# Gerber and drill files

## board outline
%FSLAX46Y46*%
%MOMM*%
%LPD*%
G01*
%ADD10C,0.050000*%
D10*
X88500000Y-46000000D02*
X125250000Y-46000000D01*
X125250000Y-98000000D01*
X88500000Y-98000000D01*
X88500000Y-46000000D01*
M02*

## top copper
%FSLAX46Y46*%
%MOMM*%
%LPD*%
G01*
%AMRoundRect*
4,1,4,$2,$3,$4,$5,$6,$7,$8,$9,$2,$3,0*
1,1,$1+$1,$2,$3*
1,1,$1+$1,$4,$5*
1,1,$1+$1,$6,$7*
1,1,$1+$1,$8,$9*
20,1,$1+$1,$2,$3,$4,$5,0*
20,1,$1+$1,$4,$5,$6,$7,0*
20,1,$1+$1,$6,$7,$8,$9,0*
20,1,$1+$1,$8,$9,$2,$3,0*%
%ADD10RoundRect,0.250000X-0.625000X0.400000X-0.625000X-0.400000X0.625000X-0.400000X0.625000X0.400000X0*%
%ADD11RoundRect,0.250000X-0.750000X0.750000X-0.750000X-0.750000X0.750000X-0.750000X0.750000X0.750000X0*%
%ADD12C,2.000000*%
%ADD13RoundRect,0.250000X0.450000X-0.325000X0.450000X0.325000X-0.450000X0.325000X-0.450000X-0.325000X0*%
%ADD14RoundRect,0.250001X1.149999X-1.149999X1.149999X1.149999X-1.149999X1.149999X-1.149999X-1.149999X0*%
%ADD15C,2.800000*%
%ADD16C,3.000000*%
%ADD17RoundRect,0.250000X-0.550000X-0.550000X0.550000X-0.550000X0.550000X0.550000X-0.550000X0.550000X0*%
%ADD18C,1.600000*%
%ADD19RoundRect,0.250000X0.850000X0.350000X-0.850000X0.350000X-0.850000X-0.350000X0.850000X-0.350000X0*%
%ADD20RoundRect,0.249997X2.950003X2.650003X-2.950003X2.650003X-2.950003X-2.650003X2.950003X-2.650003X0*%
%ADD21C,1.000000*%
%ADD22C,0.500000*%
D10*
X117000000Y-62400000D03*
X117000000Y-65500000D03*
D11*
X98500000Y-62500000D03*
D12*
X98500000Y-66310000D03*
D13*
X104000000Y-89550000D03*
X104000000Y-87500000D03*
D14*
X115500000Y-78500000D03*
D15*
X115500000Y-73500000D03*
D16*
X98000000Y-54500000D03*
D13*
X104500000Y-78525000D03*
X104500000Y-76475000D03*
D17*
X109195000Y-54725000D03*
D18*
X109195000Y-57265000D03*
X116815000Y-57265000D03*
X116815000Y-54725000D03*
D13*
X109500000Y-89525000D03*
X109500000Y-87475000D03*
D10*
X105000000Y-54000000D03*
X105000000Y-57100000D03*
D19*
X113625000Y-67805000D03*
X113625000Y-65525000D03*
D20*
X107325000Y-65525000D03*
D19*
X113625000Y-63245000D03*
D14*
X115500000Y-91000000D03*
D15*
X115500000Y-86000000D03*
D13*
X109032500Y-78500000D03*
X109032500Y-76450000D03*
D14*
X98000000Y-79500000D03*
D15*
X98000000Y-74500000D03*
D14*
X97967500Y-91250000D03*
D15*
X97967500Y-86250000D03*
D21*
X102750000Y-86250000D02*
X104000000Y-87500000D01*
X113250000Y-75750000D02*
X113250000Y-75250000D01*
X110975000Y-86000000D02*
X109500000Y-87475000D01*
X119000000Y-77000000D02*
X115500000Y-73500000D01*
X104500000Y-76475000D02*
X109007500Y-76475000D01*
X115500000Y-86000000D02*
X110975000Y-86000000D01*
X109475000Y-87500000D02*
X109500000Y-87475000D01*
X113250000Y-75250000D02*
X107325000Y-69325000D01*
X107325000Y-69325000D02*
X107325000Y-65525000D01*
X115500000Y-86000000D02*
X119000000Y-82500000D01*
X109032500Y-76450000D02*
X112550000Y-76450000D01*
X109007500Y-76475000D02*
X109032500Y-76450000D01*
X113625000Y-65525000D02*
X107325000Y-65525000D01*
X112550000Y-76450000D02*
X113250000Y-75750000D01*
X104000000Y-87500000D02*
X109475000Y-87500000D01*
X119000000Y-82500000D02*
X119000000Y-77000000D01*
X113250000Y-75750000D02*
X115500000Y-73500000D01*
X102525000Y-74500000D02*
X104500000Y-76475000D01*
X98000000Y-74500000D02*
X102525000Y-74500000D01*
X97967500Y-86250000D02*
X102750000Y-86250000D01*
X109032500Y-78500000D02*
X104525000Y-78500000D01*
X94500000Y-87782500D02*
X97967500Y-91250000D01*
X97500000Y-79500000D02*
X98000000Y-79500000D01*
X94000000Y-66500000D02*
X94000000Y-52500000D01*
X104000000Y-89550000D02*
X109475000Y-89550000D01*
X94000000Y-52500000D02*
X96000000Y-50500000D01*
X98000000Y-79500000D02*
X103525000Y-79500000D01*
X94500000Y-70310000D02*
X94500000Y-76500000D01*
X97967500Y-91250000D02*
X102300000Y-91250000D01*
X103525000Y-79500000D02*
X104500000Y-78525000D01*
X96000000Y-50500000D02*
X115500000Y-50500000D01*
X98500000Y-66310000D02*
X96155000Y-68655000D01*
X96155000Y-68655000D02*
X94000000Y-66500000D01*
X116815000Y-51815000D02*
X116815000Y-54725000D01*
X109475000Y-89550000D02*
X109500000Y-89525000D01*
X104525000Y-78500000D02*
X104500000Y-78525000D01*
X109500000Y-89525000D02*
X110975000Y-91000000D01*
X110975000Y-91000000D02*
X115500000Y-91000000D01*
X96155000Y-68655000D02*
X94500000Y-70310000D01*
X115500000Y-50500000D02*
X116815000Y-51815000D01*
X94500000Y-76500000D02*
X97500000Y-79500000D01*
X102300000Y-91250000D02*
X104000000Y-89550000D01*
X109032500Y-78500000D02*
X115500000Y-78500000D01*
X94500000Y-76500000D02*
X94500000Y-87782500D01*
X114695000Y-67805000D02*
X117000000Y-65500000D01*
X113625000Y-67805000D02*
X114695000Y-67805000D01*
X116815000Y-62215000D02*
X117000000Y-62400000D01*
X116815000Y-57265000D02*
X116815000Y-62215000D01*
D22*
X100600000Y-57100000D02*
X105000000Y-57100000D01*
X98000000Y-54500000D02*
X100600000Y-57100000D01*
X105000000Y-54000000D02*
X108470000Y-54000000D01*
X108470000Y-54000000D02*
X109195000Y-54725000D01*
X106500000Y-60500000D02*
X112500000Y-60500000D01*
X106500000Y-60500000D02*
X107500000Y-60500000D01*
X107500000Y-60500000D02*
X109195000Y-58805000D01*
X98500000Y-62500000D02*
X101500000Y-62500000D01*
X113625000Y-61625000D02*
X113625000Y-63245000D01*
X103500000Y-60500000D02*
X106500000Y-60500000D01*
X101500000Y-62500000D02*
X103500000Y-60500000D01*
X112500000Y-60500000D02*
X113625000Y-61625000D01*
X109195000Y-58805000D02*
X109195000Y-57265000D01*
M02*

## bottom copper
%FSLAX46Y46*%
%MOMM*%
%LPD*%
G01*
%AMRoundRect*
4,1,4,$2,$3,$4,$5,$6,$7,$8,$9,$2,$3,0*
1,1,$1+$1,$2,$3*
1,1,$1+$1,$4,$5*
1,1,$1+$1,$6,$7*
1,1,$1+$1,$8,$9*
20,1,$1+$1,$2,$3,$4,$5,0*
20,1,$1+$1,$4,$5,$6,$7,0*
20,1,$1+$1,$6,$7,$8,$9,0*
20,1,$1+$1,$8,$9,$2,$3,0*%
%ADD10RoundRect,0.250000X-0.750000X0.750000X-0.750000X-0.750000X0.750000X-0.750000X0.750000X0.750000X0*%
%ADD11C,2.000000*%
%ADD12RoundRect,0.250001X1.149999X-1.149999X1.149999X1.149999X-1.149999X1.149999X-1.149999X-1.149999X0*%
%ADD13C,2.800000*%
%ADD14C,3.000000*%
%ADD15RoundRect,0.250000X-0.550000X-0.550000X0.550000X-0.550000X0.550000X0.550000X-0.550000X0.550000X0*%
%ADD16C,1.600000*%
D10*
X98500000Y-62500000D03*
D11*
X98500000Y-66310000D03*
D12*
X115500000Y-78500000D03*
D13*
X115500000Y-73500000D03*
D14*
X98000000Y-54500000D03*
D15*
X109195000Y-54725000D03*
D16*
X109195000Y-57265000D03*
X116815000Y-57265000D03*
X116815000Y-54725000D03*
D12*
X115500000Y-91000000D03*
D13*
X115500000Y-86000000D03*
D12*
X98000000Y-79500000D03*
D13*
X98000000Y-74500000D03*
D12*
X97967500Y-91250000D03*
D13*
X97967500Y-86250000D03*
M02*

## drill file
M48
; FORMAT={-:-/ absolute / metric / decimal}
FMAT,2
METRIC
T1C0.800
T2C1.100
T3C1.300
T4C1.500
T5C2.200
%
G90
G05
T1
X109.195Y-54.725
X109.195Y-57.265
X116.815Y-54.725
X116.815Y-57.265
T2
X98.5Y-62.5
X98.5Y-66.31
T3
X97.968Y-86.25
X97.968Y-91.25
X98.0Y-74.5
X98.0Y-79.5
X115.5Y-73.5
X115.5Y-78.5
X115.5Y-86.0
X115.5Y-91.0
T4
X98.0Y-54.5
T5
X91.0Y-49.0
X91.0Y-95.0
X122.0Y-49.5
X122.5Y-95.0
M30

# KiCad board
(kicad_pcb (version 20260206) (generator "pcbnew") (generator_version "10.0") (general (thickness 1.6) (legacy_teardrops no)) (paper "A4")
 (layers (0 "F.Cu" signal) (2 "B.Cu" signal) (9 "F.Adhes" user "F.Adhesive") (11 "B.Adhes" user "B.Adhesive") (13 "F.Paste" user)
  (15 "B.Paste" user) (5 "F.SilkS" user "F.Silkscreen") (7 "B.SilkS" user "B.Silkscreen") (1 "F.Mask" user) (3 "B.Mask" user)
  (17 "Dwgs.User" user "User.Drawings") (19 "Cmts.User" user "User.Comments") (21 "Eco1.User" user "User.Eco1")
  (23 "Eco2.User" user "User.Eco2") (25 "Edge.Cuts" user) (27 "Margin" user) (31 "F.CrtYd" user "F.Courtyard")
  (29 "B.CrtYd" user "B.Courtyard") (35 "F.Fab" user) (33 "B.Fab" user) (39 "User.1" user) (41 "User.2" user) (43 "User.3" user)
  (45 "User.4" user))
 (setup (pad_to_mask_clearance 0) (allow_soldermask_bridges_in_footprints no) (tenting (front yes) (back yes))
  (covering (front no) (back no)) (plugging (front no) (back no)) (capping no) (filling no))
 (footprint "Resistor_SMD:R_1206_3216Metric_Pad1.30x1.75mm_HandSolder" (layer "F.Cu") (at 117 63.95 -90)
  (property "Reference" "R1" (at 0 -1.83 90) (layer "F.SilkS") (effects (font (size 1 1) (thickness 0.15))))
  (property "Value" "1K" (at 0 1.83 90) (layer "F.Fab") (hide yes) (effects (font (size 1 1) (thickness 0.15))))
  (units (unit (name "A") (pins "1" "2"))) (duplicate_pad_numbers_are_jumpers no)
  (pad "1" smd roundrect (at -1.55 0 270) (size 1.3 1.75) (layers "F.Cu" "F.Mask" "F.Paste") (roundrect_rratio 0.192308)
   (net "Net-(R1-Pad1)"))
  (pad "2" smd roundrect (at 1.55 0 270) (size 1.3 1.75) (layers "F.Cu" "F.Mask" "F.Paste") (roundrect_rratio 0.192308) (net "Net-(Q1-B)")))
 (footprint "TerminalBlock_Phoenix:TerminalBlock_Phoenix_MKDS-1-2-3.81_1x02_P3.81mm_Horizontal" (layer "F.Cu") (at 98.5 62.5 -90)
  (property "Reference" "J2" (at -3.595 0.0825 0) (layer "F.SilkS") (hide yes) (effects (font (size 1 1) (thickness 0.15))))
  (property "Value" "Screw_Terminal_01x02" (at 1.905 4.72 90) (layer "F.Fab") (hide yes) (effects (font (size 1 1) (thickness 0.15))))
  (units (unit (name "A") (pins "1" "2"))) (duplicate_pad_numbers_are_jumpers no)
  (pad "1" thru_hole roundrect (at 0 0 270) (size 2 2) (drill 1.1) (layers "*.Cu" "*.Mask") (remove_unused_layers no)
   (roundrect_rratio 0.125) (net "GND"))
  (pad "2" thru_hole circle (at 3.81 0 270) (size 2 2) (drill 1.1) (layers "*.Cu" "*.Mask") (remove_unused_layers no) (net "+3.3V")))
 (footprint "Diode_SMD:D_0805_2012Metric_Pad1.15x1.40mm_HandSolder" (layer "F.Cu") (at 104 88.525 90)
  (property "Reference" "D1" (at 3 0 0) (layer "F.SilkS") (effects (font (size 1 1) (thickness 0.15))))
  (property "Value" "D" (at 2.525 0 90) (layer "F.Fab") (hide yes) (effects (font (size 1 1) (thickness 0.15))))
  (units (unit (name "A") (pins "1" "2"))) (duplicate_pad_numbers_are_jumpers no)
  (pad "1" smd roundrect (at -1.025 0 90) (size 1.15 1.4) (layers "F.Cu" "F.Mask" "F.Paste") (roundrect_rratio 0.217391) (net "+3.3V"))
  (pad "2" smd roundrect (at 1.025 0 90) (size 1.15 1.4) (layers "F.Cu" "F.Mask" "F.Paste") (roundrect_rratio 0.217391) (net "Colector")))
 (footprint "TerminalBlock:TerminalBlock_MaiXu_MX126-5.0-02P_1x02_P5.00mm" (layer "F.Cu") (at 115.5 78.5 90)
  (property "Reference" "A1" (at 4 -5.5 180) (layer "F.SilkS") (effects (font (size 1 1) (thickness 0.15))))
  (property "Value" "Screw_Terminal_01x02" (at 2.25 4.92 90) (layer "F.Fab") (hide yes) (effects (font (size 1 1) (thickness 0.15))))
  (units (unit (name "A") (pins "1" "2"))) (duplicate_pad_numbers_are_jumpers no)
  (pad "1" thru_hole roundrect (at 0 0 90) (size 2.8 2.8) (drill 1.3) (layers "*.Cu" "*.Mask") (remove_unused_layers no)
   (roundrect_rratio 0.089286) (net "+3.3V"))
  (pad "2" thru_hole circle (at 5 0 90) (size 2.8 2.8) (drill 1.3) (layers "*.Cu" "*.Mask") (remove_unused_layers no) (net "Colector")))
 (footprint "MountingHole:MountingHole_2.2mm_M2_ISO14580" (layer "F.Cu") (at 91 95)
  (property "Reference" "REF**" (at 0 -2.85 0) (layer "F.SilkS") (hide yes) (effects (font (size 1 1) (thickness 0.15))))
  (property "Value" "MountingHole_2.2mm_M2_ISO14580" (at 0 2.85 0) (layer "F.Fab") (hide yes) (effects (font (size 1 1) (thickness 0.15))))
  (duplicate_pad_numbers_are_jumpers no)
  (pad "" np_thru_hole circle (at 0 0) (size 2.2 2.2) (drill 2.2) (layers "*.Cu" "*.Mask")))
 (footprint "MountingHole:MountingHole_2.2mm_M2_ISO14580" (layer "F.Cu") (at 122 49.5)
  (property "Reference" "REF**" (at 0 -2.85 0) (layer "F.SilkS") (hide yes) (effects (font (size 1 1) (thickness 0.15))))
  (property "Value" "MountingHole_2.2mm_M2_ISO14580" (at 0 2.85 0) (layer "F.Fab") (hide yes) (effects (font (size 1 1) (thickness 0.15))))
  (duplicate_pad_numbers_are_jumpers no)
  (pad "" np_thru_hole circle (at 0 0) (size 2.2 2.2) (drill 2.2) (layers "*.Cu" "*.Mask")))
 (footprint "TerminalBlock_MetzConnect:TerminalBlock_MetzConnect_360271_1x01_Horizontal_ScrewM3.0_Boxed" (layer "F.Cu") (at 98 54.5 180)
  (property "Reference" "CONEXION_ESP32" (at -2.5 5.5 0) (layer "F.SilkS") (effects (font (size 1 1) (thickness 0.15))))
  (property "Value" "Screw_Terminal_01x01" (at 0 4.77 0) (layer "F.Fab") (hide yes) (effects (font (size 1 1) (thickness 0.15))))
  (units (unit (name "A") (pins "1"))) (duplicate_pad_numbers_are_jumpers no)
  (pad "1" thru_hole circle (at 0 0 180) (size 3 3) (drill 1.5) (layers "*.Cu" "*.Mask") (remove_unused_layers no)
   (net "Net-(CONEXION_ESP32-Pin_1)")))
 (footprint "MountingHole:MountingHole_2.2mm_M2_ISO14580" (layer "F.Cu") (at 91 49)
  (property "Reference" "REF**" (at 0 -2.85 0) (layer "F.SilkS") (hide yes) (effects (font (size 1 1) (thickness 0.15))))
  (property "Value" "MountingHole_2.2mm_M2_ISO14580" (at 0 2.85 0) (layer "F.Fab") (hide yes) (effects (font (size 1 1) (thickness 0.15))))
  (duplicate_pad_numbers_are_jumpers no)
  (pad "" np_thru_hole circle (at 0 0) (size 2.2 2.2) (drill 2.2) (layers "*.Cu" "*.Mask")))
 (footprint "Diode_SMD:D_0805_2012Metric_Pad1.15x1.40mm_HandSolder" (layer "F.Cu") (at 104.5 77.5 90)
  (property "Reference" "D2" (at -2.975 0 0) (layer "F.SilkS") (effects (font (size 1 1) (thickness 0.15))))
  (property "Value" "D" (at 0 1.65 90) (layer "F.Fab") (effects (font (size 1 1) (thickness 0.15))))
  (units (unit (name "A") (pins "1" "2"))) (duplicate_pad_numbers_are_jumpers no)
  (pad "1" smd roundrect (at -1.025 0 90) (size 1.15 1.4) (layers "F.Cu" "F.Mask" "F.Paste") (roundrect_rratio 0.217391) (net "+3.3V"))
  (pad "2" smd roundrect (at 1.025 0 90) (size 1.15 1.4) (layers "F.Cu" "F.Mask" "F.Paste") (roundrect_rratio 0.217391) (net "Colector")))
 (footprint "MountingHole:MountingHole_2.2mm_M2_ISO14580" (layer "F.Cu") (at 122.5 95)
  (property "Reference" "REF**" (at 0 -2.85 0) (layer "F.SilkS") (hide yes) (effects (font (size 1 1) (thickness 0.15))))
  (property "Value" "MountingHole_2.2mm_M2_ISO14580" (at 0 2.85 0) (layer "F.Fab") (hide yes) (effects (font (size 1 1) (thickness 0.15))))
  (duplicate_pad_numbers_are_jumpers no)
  (pad "" np_thru_hole circle (at 0 0) (size 2.2 2.2) (drill 2.2) (layers "*.Cu" "*.Mask")))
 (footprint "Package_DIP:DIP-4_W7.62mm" (layer "F.Cu") (at 109.195 54.725)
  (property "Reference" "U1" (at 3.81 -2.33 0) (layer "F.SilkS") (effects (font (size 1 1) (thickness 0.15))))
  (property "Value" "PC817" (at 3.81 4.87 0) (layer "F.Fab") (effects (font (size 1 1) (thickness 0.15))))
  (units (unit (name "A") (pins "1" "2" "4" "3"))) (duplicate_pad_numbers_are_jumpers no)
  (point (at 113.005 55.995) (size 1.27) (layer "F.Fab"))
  (pad "1" thru_hole roundrect (at 0 0) (size 1.6 1.6) (drill 0.8) (layers "*.Cu" "*.Mask") (remove_unused_layers no)
   (roundrect_rratio 0.15625) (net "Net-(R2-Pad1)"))
  (pad "2" thru_hole circle (at 0 2.54) (size 1.6 1.6) (drill 0.8) (layers "*.Cu" "*.Mask") (remove_unused_layers no) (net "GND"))
  (pad "3" thru_hole circle (at 7.62 2.54) (size 1.6 1.6) (drill 0.8) (layers "*.Cu" "*.Mask") (remove_unused_layers no)
   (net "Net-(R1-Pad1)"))
  (pad "4" thru_hole circle (at 7.62 0) (size 1.6 1.6) (drill 0.8) (layers "*.Cu" "*.Mask") (remove_unused_layers no) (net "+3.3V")))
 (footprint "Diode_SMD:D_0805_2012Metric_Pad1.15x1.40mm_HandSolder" (layer "F.Cu") (at 109.5 88.5 90)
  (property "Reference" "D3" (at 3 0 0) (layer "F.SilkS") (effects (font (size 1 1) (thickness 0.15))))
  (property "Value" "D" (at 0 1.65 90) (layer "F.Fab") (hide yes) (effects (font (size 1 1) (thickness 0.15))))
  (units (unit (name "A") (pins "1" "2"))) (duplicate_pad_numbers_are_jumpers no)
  (pad "1" smd roundrect (at -1.025 0 90) (size 1.15 1.4) (layers "F.Cu" "F.Mask" "F.Paste") (roundrect_rratio 0.217391) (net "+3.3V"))
  (pad "2" smd roundrect (at 1.025 0 90) (size 1.15 1.4) (layers "F.Cu" "F.Mask" "F.Paste") (roundrect_rratio 0.217391) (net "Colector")))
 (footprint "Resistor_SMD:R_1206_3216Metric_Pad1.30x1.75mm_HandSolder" (layer "F.Cu") (at 105 55.55 -90)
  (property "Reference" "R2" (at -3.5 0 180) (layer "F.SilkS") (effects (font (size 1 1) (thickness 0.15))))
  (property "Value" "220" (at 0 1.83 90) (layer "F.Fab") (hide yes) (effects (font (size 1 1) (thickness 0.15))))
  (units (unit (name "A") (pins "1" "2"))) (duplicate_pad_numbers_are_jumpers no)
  (pad "1" smd roundrect (at -1.55 0 270) (size 1.3 1.75) (layers "F.Cu" "F.Mask" "F.Paste") (roundrect_rratio 0.192308)
   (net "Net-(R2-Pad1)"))
  (pad "2" smd roundrect (at 1.55 0 270) (size 1.3 1.75) (layers "F.Cu" "F.Mask" "F.Paste") (roundrect_rratio 0.192308)
   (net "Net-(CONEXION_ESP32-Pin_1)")))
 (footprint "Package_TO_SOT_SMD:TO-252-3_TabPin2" (layer "F.Cu") (at 108.585 65.525 180)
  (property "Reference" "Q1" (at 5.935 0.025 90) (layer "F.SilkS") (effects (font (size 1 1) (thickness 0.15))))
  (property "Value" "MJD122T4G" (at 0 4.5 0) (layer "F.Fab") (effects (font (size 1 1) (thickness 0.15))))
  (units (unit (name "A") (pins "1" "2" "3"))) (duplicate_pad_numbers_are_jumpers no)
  (pad "" smd roundrect (at -0.415 -1.525 180) (size 3.05 2.75) (layers "F.Paste") (roundrect_rratio 0.090909))
  (pad "" smd roundrect (at -0.415 1.525 180) (size 3.05 2.75) (layers "F.Paste") (roundrect_rratio 0.090909))
  (pad "" smd roundrect (at 2.935 -1.525 180) (size 3.05 2.75) (layers "F.Paste") (roundrect_rratio 0.090909))
  (pad "" smd roundrect (at 2.935 1.525 180) (size 3.05 2.75) (layers "F.Paste") (roundrect_rratio 0.090909))
  (pad "1" smd roundrect (at -5.04 -2.28 180) (size 2.2 1.2) (layers "F.Cu" "F.Mask" "F.Paste") (roundrect_rratio 0.208333)
   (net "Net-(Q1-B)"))
  (pad "2" smd roundrect (at -5.04 0 180) (size 2.2 1.2) (layers "F.Cu" "F.Mask" "F.Paste") (roundrect_rratio 0.208333) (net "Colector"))
  (pad "2" smd roundrect (at 1.26 0 180) (size 6.4 5.8) (layers "F.Cu" "F.Mask") (roundrect_rratio 0.043103) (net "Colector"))
  (pad "3" smd roundrect (at -5.04 2.28 180) (size 2.2 1.2) (layers "F.Cu" "F.Mask" "F.Paste") (roundrect_rratio 0.208333) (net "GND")))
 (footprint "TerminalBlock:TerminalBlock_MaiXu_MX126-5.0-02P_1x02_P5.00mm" (layer "F.Cu") (at 115.5 91 90)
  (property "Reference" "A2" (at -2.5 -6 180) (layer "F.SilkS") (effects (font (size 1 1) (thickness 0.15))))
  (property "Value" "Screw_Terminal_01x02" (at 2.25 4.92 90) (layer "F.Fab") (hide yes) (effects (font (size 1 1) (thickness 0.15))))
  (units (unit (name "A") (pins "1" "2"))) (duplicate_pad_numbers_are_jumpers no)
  (pad "1" thru_hole roundrect (at 0 0 90) (size 2.8 2.8) (drill 1.3) (layers "*.Cu" "*.Mask") (remove_unused_layers no)
   (roundrect_rratio 0.089286) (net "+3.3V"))
  (pad "2" thru_hole circle (at 5 0 90) (size 2.8 2.8) (drill 1.3) (layers "*.Cu" "*.Mask") (remove_unused_layers no) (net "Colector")))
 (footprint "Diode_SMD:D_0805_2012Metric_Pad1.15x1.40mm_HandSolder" (layer "F.Cu") (at 109.0325 77.475 90)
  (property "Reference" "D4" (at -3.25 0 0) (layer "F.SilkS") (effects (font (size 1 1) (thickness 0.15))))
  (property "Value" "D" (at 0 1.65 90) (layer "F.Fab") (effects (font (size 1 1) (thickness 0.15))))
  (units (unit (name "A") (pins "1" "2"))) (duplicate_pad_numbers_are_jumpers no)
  (pad "1" smd roundrect (at -1.025 0 90) (size 1.15 1.4) (layers "F.Cu" "F.Mask" "F.Paste") (roundrect_rratio 0.217391) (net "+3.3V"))
  (pad "2" smd roundrect (at 1.025 0 90) (size 1.15 1.4) (layers "F.Cu" "F.Mask" "F.Paste") (roundrect_rratio 0.217391) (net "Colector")))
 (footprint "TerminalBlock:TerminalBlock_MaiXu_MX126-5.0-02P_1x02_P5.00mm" (layer "F.Cu") (at 98 79.5 90)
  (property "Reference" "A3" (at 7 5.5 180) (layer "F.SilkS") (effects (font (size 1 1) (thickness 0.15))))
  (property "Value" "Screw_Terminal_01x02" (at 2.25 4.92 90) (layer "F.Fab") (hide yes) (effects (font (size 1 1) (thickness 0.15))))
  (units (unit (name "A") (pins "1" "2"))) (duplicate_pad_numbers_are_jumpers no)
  (pad "1" thru_hole roundrect (at 0 0 90) (size 2.8 2.8) (drill 1.3) (layers "*.Cu" "*.Mask") (remove_unused_layers no)
   (roundrect_rratio 0.089286) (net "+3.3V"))
  (pad "2" thru_hole circle (at 5 0 90) (size 2.8 2.8) (drill 1.3) (layers "*.Cu" "*.Mask") (remove_unused_layers no) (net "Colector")))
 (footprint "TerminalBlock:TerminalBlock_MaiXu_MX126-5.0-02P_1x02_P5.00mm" (layer "F.Cu") (at 97.9675 91.25 90)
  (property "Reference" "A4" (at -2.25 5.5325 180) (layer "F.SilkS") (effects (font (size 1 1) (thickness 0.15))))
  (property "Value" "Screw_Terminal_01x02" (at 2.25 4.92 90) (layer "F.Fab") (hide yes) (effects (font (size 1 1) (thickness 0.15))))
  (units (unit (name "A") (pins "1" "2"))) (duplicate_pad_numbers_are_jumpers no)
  (pad "1" thru_hole roundrect (at 0 0 90) (size 2.8 2.8) (drill 1.3) (layers "*.Cu" "*.Mask") (remove_unused_layers no)
   (roundrect_rratio 0.089286) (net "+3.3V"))
  (pad "2" thru_hole circle (at 5 0 90) (size 2.8 2.8) (drill 1.3) (layers "*.Cu" "*.Mask") (remove_unused_layers no) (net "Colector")))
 (gr_rect (start 88.5 46) (end 125.25 98) (stroke (width 0.05) (type default)) (fill no) (layer "Edge.Cuts"))
 (segment (start 102.75 86.25) (end 104 87.5) (width 1) (layer "F.Cu") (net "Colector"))
 (segment (start 113.25 75.75) (end 113.25 75.25) (width 1) (layer "F.Cu") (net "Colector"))
 (segment (start 110.975 86) (end 109.5 87.475) (width 1) (layer "F.Cu") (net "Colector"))
 (segment (start 119 77) (end 115.5 73.5) (width 1) (layer "F.Cu") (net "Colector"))
 (segment (start 104.5 76.475) (end 109.0075 76.475) (width 1) (layer "F.Cu") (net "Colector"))
 (segment (start 115.5 86) (end 110.975 86) (width 1) (layer "F.Cu") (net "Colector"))
 (segment (start 109.475 87.5) (end 109.5 87.475) (width 1) (layer "F.Cu") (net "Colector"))
 (segment (start 113.25 75.25) (end 107.325 69.325) (width 1) (layer "F.Cu") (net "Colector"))
 (segment (start 107.325 69.325) (end 107.325 65.525) (width 1) (layer "F.Cu") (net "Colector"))
 (segment (start 115.5 86) (end 119 82.5) (width 1) (layer "F.Cu") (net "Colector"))
 (segment (start 109.0325 76.45) (end 112.55 76.45) (width 1) (layer "F.Cu") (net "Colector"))
 (segment (start 109.0075 76.475) (end 109.0325 76.45) (width 1) (layer "F.Cu") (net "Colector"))
 (segment (start 113.625 65.525) (end 107.325 65.525) (width 1) (layer "F.Cu") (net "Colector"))
 (segment (start 112.55 76.45) (end 113.25 75.75) (width 1) (layer "F.Cu") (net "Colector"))
 (segment (start 104 87.5) (end 109.475 87.5) (width 1) (layer "F.Cu") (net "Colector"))
 (segment (start 119 82.5) (end 119 77) (width 1) (layer "F.Cu") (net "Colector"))
 (segment (start 113.25 75.75) (end 115.5 73.5) (width 1) (layer "F.Cu") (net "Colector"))
 (segment (start 102.525 74.5) (end 104.5 76.475) (width 1) (layer "F.Cu") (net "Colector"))
 (segment (start 98 74.5) (end 102.525 74.5) (width 1) (layer "F.Cu") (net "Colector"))
 (segment (start 97.9675 86.25) (end 102.75 86.25) (width 1) (layer "F.Cu") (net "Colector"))
 (segment (start 109.0325 78.5) (end 104.525 78.5) (width 1) (layer "F.Cu") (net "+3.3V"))
 (segment (start 94.5 87.7825) (end 97.9675 91.25) (width 1) (layer "F.Cu") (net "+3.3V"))
 (segment (start 97.5 79.5) (end 98 79.5) (width 1) (layer "F.Cu") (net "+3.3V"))
 (segment (start 94 66.5) (end 94 52.5) (width 1) (layer "F.Cu") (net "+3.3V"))
 (segment (start 104 89.55) (end 109.475 89.55) (width 1) (layer "F.Cu") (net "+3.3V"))
 (segment (start 94 52.5) (end 96 50.5) (width 1) (layer "F.Cu") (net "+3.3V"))
 (segment (start 98 79.5) (end 103.525 79.5) (width 1) (layer "F.Cu") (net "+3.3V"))
 (segment (start 94.5 70.31) (end 94.5 76.5) (width 1) (layer "F.Cu") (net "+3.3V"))
 (segment (start 97.9675 91.25) (end 102.3 91.25) (width 1) (layer "F.Cu") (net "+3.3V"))
 (segment (start 103.525 79.5) (end 104.5 78.525) (width 1) (layer "F.Cu") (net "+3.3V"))
 (segment (start 96 50.5) (end 115.5 50.5) (width 1) (layer "F.Cu") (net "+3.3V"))
 (segment (start 98.5 66.31) (end 96.155 68.655) (width 1) (layer "F.Cu") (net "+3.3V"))
 (segment (start 96.155 68.655) (end 94 66.5) (width 1) (layer "F.Cu") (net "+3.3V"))
 (segment (start 116.815 51.815) (end 116.815 54.725) (width 1) (layer "F.Cu") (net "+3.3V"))
 (segment (start 109.475 89.55) (end 109.5 89.525) (width 1) (layer "F.Cu") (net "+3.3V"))
 (segment (start 104.525 78.5) (end 104.5 78.525) (width 1) (layer "F.Cu") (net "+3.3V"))
 (segment (start 109.5 89.525) (end 110.975 91) (width 1) (layer "F.Cu") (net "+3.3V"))
 (segment (start 110.975 91) (end 115.5 91) (width 1) (layer "F.Cu") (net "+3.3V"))
 (segment (start 96.155 68.655) (end 94.5 70.31) (width 1) (layer "F.Cu") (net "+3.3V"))
 (segment (start 115.5 50.5) (end 116.815 51.815) (width 1) (layer "F.Cu") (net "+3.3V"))
 (segment (start 94.5 76.5) (end 97.5 79.5) (width 1) (layer "F.Cu") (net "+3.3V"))
 (segment (start 102.3 91.25) (end 104 89.55) (width 1) (layer "F.Cu") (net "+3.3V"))
 (segment (start 109.0325 78.5) (end 115.5 78.5) (width 1) (layer "F.Cu") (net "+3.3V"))
 (segment (start 94.5 76.5) (end 94.5 87.7825) (width 1) (layer "F.Cu") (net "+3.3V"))
 (segment (start 114.695 67.805) (end 117 65.5) (width 1) (layer "F.Cu") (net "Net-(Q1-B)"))
 (segment (start 113.625 67.805) (end 114.695 67.805) (width 1) (layer "F.Cu") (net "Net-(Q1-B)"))
 (segment (start 116.815 62.215) (end 117 62.4) (width 1) (layer "F.Cu") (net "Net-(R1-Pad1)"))
 (segment (start 116.815 57.265) (end 116.815 62.215) (width 1) (layer "F.Cu") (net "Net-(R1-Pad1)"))
 (segment (start 100.6 57.1) (end 105 57.1) (width 0.5) (layer "F.Cu") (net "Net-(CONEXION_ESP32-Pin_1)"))
 (segment (start 98 54.5) (end 100.6 57.1) (width 0.5) (layer "F.Cu") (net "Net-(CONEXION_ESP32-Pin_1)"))
 (segment (start 105 54) (end 108.47 54) (width 0.5) (layer "F.Cu") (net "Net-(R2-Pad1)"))
 (segment (start 108.47 54) (end 109.195 54.725) (width 0.5) (layer "F.Cu") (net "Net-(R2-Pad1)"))
 (segment (start 106.5 60.5) (end 112.5 60.5) (width 0.5) (layer "F.Cu") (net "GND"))
 (segment (start 106.5 60.5) (end 107.5 60.5) (width 0.5) (layer "F.Cu") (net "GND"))
 (segment (start 107.5 60.5) (end 109.195 58.805) (width 0.5) (layer "F.Cu") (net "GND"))
 (segment (start 98.5 62.5) (end 101.5 62.5) (width 0.5) (layer "F.Cu") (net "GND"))
 (segment (start 113.625 61.625) (end 113.625 63.245) (width 0.5) (layer "F.Cu") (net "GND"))
 (segment (start 103.5 60.5) (end 106.5 60.5) (width 0.5) (layer "F.Cu") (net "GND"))
 (segment (start 101.5 62.5) (end 103.5 60.5) (width 0.5) (layer "F.Cu") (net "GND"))
 (segment (start 112.5 60.5) (end 113.625 61.625) (width 0.5) (layer "F.Cu") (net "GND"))
 (segment (start 109.195 58.805) (end 109.195 57.265) (width 0.5) (layer "F.Cu") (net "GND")))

